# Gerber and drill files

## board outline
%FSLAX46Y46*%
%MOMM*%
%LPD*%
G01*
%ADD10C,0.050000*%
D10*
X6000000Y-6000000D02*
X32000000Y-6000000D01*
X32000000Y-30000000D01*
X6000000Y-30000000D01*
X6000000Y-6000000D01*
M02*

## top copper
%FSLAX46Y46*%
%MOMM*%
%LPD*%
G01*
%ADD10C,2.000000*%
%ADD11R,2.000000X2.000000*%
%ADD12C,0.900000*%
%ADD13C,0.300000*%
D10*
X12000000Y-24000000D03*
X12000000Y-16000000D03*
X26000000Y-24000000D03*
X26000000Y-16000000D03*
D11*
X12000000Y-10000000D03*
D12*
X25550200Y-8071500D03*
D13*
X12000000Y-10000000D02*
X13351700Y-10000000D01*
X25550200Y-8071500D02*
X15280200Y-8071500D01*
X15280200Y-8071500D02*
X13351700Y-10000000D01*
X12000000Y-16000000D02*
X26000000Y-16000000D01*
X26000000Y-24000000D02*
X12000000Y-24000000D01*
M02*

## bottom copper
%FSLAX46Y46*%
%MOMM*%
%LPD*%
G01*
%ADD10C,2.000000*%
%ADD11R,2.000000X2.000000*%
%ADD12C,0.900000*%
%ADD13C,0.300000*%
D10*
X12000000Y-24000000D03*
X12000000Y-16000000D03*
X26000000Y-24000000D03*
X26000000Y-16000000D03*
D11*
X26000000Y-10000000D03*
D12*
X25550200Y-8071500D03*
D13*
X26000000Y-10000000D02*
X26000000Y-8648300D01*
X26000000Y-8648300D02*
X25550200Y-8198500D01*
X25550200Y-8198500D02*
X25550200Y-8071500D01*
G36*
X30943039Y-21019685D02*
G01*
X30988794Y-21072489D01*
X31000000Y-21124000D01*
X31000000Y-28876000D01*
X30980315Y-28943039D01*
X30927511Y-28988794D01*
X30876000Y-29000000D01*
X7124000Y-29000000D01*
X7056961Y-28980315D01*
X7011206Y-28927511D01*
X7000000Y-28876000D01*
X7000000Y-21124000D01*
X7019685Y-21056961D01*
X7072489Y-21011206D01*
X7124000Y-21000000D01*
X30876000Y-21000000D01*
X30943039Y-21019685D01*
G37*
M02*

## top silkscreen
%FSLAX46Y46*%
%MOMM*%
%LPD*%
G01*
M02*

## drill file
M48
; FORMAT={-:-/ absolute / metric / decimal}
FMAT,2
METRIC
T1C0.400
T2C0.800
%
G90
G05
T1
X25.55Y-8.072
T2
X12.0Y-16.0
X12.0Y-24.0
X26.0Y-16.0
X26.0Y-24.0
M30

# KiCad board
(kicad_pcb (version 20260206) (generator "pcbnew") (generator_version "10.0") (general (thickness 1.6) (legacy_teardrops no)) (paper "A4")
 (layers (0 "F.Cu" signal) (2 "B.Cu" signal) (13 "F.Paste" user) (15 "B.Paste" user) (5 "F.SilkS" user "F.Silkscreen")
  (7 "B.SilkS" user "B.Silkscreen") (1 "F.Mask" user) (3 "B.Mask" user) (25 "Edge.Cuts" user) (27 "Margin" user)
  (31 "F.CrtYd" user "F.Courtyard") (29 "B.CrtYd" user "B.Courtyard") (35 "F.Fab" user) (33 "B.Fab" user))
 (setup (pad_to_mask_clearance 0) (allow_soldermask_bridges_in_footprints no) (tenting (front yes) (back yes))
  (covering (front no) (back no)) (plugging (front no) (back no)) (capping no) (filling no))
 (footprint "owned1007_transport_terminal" (layer "F.Cu") (at 12 24)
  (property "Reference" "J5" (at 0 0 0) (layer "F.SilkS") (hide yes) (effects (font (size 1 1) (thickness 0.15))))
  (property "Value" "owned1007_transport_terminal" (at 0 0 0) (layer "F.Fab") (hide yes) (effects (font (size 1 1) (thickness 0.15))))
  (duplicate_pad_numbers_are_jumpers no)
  (pad "1" thru_hole circle (at 0 0) (size 2 2) (drill 0.8) (layers "*.Cu" "*.Mask") (remove_unused_layers no) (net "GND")))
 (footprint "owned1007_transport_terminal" (layer "F.Cu") (at 12 16)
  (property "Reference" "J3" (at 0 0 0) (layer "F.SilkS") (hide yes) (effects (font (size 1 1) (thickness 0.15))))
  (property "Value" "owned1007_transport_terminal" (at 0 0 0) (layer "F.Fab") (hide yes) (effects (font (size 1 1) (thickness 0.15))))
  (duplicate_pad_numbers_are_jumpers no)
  (pad "1" thru_hole circle (at 0 0) (size 2 2) (drill 0.8) (layers "*.Cu" "*.Mask") (remove_unused_layers no) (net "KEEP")))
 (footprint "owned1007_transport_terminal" (layer "F.Cu") (at 26 24)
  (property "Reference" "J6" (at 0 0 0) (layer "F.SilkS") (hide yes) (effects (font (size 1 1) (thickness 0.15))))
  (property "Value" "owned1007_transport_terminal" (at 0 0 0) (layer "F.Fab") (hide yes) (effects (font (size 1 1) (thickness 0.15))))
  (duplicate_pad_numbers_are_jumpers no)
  (pad "1" thru_hole circle (at 0 0) (size 2 2) (drill 0.8) (layers "*.Cu" "*.Mask") (remove_unused_layers no) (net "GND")))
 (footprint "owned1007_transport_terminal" (layer "F.Cu") (at 26 16)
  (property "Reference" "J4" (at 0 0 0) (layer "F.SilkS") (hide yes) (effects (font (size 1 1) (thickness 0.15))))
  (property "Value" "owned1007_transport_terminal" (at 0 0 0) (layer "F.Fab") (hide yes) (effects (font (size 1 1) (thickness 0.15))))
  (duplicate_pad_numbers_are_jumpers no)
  (pad "1" thru_hole circle (at 0 0) (size 2 2) (drill 0.8) (layers "*.Cu" "*.Mask") (remove_unused_layers no) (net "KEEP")))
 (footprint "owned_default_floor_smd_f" (layer "F.Cu") (at 12 10)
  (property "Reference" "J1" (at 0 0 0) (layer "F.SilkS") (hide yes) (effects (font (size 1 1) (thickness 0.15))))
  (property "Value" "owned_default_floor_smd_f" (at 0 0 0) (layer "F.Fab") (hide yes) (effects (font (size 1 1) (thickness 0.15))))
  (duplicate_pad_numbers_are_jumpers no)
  (pad "1" smd rect (at 0 0) (size 2 2) (layers "F.Cu" "F.Mask" "F.Paste") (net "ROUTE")))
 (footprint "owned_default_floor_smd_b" (layer "B.Cu") (at 26 10)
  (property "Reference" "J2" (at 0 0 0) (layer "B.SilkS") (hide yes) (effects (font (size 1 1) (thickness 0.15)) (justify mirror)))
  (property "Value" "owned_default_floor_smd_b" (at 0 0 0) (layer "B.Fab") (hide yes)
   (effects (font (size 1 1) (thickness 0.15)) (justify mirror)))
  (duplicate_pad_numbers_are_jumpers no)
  (pad "1" smd rect (at 0 0) (size 2 2) (layers "B.Cu" "B.Mask" "B.Paste") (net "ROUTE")))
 (gr_rect (start 6 6) (end 32 30) (stroke (width 0.05) (type default)) (fill no) (layer "Edge.Cuts"))
 (segment (start 12 10) (end 13.3517 10) (width 0.3) (layer "F.Cu") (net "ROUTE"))
 (segment (start 25.5502 8.0715) (end 15.2802 8.0715) (width 0.3) (layer "F.Cu") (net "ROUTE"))
 (segment (start 15.2802 8.0715) (end 13.3517 10) (width 0.3) (layer "F.Cu") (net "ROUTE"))
 (via (at 25.5502 8.0715) (size 0.9) (drill 0.4) (layers "F.Cu" "B.Cu") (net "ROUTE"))
 (segment (start 26 10) (end 26 8.6483) (width 0.3) (layer "B.Cu") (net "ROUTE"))
 (segment (start 26 8.6483) (end 25.5502 8.1985) (width 0.3) (layer "B.Cu") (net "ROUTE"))
 (segment (start 25.5502 8.1985) (end 25.5502 8.0715) (width 0.3) (layer "B.Cu") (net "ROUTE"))
 (segment (start 12 16) (end 26 16) (width 0.3) (locked yes) (layer "F.Cu") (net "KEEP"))
 (segment (start 26 24) (end 12 24) (width 0.3) (layer "F.Cu") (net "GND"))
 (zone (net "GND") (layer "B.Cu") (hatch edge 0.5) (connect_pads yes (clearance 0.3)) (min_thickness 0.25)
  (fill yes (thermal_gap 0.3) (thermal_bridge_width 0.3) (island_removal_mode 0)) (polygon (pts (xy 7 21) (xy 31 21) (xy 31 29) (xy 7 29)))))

